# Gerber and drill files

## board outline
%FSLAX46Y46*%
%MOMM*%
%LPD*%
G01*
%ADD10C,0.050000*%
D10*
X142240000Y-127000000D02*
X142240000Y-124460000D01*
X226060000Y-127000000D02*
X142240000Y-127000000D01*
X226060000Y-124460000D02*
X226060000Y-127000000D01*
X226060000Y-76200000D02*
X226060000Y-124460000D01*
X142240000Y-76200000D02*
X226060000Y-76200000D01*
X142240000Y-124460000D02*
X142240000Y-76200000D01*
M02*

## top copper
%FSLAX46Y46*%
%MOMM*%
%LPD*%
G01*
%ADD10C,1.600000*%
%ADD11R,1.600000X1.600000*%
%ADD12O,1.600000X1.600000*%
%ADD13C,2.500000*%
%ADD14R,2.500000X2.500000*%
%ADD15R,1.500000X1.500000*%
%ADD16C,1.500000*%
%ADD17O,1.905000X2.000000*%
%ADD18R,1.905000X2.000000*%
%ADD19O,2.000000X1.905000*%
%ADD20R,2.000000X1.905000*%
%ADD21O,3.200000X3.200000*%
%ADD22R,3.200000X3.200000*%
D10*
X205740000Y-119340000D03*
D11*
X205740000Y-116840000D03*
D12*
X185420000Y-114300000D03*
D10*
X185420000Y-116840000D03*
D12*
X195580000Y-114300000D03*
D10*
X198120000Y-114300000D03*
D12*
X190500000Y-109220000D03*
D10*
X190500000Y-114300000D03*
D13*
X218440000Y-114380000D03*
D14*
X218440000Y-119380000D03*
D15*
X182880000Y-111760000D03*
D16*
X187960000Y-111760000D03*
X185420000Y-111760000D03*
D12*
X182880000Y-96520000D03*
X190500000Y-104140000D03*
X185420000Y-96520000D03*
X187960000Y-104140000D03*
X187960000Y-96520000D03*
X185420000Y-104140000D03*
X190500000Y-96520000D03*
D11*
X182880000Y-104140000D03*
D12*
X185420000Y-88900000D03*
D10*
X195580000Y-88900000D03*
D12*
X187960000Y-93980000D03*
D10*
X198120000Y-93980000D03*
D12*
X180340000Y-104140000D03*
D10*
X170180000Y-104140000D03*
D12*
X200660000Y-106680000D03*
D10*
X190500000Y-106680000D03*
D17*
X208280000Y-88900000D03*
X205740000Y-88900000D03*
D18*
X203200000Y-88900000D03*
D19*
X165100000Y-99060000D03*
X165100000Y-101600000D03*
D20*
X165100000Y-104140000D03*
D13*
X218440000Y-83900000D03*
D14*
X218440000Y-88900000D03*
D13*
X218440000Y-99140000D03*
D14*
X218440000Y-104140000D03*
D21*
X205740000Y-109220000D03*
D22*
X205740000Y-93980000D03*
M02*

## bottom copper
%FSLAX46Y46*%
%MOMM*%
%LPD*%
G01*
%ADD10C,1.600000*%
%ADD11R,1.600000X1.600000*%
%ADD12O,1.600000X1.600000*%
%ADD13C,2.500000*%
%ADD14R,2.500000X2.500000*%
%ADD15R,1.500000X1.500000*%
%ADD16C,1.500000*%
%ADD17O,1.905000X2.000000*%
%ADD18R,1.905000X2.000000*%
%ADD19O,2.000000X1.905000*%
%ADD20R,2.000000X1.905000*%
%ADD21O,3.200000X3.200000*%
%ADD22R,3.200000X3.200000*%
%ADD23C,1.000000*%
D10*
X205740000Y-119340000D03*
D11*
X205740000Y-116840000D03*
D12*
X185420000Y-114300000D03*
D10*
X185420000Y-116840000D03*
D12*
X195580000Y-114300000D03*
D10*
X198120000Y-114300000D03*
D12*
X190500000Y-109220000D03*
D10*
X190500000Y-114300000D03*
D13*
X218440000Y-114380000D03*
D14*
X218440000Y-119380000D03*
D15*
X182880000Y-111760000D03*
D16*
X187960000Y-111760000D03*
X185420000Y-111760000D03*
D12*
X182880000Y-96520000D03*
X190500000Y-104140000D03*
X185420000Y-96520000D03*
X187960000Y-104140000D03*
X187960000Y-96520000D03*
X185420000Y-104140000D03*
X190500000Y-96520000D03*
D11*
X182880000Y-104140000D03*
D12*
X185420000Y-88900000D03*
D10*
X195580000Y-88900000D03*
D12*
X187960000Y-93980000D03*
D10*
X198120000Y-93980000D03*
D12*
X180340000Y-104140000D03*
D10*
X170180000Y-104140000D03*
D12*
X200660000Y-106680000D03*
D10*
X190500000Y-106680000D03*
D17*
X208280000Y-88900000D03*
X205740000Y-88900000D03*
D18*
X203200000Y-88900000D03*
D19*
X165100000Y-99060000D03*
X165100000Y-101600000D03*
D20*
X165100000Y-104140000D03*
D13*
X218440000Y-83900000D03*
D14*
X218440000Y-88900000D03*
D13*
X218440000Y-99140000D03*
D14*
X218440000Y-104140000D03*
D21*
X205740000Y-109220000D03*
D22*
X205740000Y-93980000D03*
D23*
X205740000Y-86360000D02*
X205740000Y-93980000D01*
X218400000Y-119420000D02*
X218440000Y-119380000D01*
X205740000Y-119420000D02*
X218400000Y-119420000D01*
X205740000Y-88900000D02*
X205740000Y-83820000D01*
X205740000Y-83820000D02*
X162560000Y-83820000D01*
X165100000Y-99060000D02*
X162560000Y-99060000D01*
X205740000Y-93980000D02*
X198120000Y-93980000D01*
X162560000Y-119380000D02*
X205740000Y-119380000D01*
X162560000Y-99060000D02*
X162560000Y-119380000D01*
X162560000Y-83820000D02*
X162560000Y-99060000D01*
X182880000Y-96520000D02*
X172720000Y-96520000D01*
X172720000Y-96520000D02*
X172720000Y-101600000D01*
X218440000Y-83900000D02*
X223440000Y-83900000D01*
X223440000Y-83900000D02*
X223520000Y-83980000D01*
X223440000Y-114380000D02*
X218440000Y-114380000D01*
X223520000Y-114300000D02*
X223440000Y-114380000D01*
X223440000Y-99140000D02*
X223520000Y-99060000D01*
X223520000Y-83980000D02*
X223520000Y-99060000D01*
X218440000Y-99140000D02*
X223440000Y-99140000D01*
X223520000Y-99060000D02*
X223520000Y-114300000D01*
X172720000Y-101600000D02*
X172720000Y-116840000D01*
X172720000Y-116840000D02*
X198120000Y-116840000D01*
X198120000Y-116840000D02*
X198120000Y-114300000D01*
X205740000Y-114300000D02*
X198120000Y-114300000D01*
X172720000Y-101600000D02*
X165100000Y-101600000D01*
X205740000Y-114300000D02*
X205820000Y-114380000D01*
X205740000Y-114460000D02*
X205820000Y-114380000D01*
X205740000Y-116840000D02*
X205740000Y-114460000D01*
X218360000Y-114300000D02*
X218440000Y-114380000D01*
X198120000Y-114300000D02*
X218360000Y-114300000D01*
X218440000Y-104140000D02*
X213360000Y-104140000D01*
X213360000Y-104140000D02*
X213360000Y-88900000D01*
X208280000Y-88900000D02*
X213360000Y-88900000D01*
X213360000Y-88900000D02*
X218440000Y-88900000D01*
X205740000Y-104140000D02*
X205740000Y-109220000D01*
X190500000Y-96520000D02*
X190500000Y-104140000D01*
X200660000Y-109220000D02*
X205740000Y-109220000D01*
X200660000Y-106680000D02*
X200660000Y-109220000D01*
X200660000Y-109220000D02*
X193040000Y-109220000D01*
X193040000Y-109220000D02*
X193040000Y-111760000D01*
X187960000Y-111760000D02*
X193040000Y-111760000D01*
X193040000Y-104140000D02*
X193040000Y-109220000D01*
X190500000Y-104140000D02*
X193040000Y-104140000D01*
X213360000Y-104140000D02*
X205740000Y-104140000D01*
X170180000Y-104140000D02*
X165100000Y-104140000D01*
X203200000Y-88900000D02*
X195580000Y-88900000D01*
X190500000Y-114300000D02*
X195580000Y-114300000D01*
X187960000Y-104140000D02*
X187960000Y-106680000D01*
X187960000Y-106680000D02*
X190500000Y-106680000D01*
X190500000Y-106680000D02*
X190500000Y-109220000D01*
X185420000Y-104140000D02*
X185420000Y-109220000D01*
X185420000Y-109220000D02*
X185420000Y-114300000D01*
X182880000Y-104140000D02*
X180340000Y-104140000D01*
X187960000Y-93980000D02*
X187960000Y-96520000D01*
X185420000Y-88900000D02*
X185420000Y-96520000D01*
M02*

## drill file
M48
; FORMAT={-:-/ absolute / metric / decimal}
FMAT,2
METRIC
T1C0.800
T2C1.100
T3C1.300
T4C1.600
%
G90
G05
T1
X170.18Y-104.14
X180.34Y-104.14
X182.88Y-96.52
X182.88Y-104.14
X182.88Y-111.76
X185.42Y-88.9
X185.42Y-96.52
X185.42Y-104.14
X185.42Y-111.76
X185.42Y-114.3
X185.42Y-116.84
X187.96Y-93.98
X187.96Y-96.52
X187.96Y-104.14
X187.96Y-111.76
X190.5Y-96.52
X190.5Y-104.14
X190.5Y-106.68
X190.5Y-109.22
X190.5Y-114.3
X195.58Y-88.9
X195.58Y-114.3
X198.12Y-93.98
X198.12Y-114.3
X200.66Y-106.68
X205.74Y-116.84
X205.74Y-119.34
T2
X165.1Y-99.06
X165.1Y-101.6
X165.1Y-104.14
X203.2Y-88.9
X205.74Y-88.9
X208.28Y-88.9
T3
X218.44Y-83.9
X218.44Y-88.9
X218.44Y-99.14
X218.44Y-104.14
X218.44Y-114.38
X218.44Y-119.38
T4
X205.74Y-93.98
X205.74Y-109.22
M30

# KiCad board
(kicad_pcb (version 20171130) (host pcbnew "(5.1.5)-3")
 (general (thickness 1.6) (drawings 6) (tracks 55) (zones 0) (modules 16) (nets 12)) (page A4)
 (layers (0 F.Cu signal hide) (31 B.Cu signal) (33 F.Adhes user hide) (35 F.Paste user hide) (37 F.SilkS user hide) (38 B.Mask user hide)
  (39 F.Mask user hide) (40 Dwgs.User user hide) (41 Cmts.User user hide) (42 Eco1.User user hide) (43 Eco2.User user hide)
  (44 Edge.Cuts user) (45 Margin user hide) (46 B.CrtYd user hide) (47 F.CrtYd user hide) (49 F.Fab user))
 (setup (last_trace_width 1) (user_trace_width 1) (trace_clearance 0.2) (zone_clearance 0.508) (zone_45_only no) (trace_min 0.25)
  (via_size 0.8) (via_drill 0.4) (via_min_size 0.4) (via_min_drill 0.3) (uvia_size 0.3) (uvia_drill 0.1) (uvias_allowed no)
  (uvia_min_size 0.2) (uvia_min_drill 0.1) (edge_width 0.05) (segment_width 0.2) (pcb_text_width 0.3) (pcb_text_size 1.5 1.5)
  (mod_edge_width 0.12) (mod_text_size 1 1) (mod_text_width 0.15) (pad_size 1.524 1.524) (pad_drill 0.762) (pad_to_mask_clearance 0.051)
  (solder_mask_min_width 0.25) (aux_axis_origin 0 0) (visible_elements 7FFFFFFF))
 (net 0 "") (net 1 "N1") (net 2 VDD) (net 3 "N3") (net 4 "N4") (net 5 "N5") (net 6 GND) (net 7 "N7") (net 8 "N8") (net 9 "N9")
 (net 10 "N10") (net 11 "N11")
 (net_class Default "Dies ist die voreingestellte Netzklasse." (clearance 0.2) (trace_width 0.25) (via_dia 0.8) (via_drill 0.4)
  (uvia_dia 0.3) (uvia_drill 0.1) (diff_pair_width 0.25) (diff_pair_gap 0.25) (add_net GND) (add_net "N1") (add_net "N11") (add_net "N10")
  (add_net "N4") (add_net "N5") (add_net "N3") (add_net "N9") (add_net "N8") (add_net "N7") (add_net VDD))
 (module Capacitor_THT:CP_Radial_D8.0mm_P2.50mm (layer F.Cu) (at 205.74 116.84 270)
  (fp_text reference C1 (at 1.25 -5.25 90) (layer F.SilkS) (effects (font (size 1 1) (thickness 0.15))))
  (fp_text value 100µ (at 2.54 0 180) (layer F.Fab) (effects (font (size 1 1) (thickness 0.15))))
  (pad 2 thru_hole circle (at 2.5 0 270) (size 1.6 1.6) (drill 0.8) (layers *.Cu *.Mask) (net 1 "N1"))
  (pad 1 thru_hole rect (at 0 0 270) (size 1.6 1.6) (drill 0.8) (layers *.Cu *.Mask) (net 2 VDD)))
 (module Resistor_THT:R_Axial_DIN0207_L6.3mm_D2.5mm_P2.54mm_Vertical (layer F.Cu) (at 185.42 116.84 90)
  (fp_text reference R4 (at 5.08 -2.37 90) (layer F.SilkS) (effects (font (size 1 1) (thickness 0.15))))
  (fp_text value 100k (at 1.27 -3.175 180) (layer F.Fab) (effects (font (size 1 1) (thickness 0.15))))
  (pad 2 thru_hole oval (at 2.54 0 90) (size 1.6 1.6) (drill 0.8) (layers *.Cu *.Mask) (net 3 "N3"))
  (pad 1 thru_hole circle (at 0 0 90) (size 1.6 1.6) (drill 0.8) (layers *.Cu *.Mask) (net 2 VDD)))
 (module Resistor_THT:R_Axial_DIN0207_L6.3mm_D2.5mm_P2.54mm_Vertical (layer F.Cu) (at 198.12 114.3 180)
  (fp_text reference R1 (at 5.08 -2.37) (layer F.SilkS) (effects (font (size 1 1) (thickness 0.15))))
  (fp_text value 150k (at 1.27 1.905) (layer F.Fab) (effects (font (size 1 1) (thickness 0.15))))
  (pad 2 thru_hole oval (at 2.54 0 180) (size 1.6 1.6) (drill 0.8) (layers *.Cu *.Mask) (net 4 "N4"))
  (pad 1 thru_hole circle (at 0 0 180) (size 1.6 1.6) (drill 0.8) (layers *.Cu *.Mask) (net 2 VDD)))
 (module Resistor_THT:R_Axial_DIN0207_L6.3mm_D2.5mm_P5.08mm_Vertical (layer F.Cu) (at 190.5 114.3 90)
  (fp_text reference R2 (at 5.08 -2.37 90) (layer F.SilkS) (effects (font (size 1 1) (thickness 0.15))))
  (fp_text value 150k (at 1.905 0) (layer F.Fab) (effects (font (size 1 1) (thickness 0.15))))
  (pad 2 thru_hole oval (at 5.08 0 90) (size 1.6 1.6) (drill 0.8) (layers *.Cu *.Mask) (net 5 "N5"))
  (pad 1 thru_hole circle (at 0 0 90) (size 1.6 1.6) (drill 0.8) (layers *.Cu *.Mask) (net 4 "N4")))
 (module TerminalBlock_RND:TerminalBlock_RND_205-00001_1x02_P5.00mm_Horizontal (layer F.Cu) (at 218.44 119.38 90)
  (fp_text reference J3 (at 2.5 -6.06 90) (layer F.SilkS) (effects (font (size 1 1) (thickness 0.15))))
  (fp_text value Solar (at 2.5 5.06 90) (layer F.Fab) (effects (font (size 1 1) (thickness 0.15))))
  (pad 2 thru_hole circle (at 5 0 90) (size 2.5 2.5) (drill 1.3) (layers *.Cu *.Mask) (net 2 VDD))
  (pad 1 thru_hole rect (at 0 0 90) (size 2.5 2.5) (drill 1.3) (layers *.Cu *.Mask) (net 1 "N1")))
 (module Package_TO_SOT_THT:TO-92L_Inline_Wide (layer F.Cu) (at 182.88 111.76)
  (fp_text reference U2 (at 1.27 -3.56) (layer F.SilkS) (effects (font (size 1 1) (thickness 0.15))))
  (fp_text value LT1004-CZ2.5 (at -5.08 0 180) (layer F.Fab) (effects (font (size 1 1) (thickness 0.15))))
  (pad 1 thru_hole rect (at 0 0 90) (size 1.5 1.5) (drill 0.8) (layers *.Cu *.Mask))
  (pad 3 thru_hole circle (at 5.08 0 90) (size 1.5 1.5) (drill 0.8) (layers *.Cu *.Mask) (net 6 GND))
  (pad 2 thru_hole circle (at 2.54 0 90) (size 1.5 1.5) (drill 0.8) (layers *.Cu *.Mask) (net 3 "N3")))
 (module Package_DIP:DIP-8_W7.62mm (layer F.Cu) (at 182.88 104.14 90)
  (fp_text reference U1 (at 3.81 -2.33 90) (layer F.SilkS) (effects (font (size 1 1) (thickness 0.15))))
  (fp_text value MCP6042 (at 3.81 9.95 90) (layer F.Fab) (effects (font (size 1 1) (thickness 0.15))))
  (pad 8 thru_hole oval (at 7.62 0 90) (size 1.6 1.6) (drill 0.8) (layers *.Cu *.Mask) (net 2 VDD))
  (pad 4 thru_hole oval (at 0 7.62 90) (size 1.6 1.6) (drill 0.8) (layers *.Cu *.Mask) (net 6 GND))
  (pad 7 thru_hole oval (at 7.62 2.54 90) (size 1.6 1.6) (drill 0.8) (layers *.Cu *.Mask) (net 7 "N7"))
  (pad 3 thru_hole oval (at 0 5.08 90) (size 1.6 1.6) (drill 0.8) (layers *.Cu *.Mask) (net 5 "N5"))
  (pad 6 thru_hole oval (at 7.62 5.08 90) (size 1.6 1.6) (drill 0.8) (layers *.Cu *.Mask) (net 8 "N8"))
  (pad 2 thru_hole oval (at 0 2.54 90) (size 1.6 1.6) (drill 0.8) (layers *.Cu *.Mask) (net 3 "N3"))
  (pad 5 thru_hole oval (at 7.62 7.62 90) (size 1.6 1.6) (drill 0.8) (layers *.Cu *.Mask) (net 6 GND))
  (pad 1 thru_hole rect (at 0 0 90) (size 1.6 1.6) (drill 0.8) (layers *.Cu *.Mask) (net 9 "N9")))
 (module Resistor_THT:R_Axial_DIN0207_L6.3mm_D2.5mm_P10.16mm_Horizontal (layer F.Cu) (at 195.58 88.9 180)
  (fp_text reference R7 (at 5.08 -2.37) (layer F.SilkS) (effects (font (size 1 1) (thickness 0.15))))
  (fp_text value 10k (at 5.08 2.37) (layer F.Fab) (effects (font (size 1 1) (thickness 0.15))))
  (pad 2 thru_hole oval (at 10.16 0 180) (size 1.6 1.6) (drill 0.8) (layers *.Cu *.Mask) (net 7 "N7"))
  (pad 1 thru_hole circle (at 0 0 180) (size 1.6 1.6) (drill 0.8) (layers *.Cu *.Mask) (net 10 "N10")))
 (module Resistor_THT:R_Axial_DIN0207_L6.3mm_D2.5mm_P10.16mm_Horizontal (layer F.Cu) (at 198.12 93.98 180)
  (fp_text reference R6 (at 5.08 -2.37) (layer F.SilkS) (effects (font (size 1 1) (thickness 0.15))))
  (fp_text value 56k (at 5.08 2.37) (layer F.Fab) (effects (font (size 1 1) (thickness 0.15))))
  (pad 2 thru_hole oval (at 10.16 0 180) (size 1.6 1.6) (drill 0.8) (layers *.Cu *.Mask) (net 8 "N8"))
  (pad 1 thru_hole circle (at 0 0 180) (size 1.6 1.6) (drill 0.8) (layers *.Cu *.Mask) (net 1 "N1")))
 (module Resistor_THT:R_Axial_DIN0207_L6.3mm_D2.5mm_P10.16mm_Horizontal (layer F.Cu) (at 170.18 104.14)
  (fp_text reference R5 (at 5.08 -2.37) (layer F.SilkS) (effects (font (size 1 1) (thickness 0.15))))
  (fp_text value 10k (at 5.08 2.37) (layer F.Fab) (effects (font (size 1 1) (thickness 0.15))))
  (pad 2 thru_hole oval (at 10.16 0) (size 1.6 1.6) (drill 0.8) (layers *.Cu *.Mask) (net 9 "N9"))
  (pad 1 thru_hole circle (at 0 0) (size 1.6 1.6) (drill 0.8) (layers *.Cu *.Mask) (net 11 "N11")))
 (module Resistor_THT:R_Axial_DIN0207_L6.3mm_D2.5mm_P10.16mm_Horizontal (layer F.Cu) (at 190.5 106.68)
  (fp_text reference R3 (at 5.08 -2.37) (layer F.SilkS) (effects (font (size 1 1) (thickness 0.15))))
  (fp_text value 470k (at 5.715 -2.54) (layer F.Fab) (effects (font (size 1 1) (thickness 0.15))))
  (pad 2 thru_hole oval (at 10.16 0) (size 1.6 1.6) (drill 0.8) (layers *.Cu *.Mask) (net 6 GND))
  (pad 1 thru_hole circle (at 0 0) (size 1.6 1.6) (drill 0.8) (layers *.Cu *.Mask) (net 5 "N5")))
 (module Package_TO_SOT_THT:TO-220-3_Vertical (layer F.Cu) (at 203.2 88.9)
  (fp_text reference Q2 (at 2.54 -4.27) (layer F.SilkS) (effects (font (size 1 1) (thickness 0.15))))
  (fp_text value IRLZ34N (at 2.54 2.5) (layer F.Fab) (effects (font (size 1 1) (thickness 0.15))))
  (pad 3 thru_hole oval (at 5.08 0) (size 1.905 2) (drill 1.1) (layers *.Cu *.Mask) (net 6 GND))
  (pad 2 thru_hole oval (at 2.54 0) (size 1.905 2) (drill 1.1) (layers *.Cu *.Mask) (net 1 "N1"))
  (pad 1 thru_hole rect (at 0 0) (size 1.905 2) (drill 1.1) (layers *.Cu *.Mask) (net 10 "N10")))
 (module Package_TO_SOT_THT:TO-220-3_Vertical (layer F.Cu) (at 165.1 104.14 90)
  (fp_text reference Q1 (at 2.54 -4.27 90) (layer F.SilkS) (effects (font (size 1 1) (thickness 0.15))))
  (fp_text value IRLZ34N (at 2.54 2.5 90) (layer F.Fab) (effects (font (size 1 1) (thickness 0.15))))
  (pad 3 thru_hole oval (at 5.08 0 90) (size 1.905 2) (drill 1.1) (layers *.Cu *.Mask) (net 1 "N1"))
  (pad 2 thru_hole oval (at 2.54 0 90) (size 1.905 2) (drill 1.1) (layers *.Cu *.Mask) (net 2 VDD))
  (pad 1 thru_hole rect (at 0 0 90) (size 1.905 2) (drill 1.1) (layers *.Cu *.Mask) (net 11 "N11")))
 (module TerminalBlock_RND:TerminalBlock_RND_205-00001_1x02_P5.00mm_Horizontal (layer F.Cu) (at 218.44 88.9 90)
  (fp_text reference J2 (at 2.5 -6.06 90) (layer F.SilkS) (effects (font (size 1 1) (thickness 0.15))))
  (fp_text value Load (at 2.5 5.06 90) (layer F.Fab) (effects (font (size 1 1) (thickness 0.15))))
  (pad 2 thru_hole circle (at 5 0 90) (size 2.5 2.5) (drill 1.3) (layers *.Cu *.Mask) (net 2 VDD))
  (pad 1 thru_hole rect (at 0 0 90) (size 2.5 2.5) (drill 1.3) (layers *.Cu *.Mask) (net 6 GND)))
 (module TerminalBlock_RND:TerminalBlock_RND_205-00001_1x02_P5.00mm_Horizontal (layer F.Cu) (at 218.44 104.14 90)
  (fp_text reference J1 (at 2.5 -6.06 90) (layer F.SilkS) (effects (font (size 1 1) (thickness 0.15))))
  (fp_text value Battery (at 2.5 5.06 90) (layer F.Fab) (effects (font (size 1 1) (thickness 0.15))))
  (pad 2 thru_hole circle (at 5 0 90) (size 2.5 2.5) (drill 1.3) (layers *.Cu *.Mask) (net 2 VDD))
  (pad 1 thru_hole rect (at 0 0 90) (size 2.5 2.5) (drill 1.3) (layers *.Cu *.Mask) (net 6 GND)))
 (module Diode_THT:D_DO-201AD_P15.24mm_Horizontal (layer F.Cu) (at 205.74 93.98 270)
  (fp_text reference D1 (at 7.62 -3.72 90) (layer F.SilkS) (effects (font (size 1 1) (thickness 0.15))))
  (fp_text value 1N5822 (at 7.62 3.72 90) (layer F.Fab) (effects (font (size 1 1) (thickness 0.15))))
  (pad 2 thru_hole oval (at 15.24 0 270) (size 3.2 3.2) (drill 1.6) (layers *.Cu *.Mask) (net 6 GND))
  (pad 1 thru_hole rect (at 0 0 270) (size 3.2 3.2) (drill 1.6) (layers *.Cu *.Mask) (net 1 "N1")))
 (gr_line (start 142.24 127) (end 142.24 124.46) (layer Edge.Cuts) (width 0.05))
 (gr_line (start 226.06 127) (end 142.24 127) (layer Edge.Cuts) (width 0.05))
 (gr_line (start 226.06 124.46) (end 226.06 127) (layer Edge.Cuts) (width 0.05))
 (gr_line (start 226.06 76.2) (end 226.06 124.46) (layer Edge.Cuts) (width 0.05))
 (gr_line (start 142.24 76.2) (end 226.06 76.2) (layer Edge.Cuts) (width 0.05))
 (gr_line (start 142.24 124.46) (end 142.24 76.2) (layer Edge.Cuts) (width 0.05))
 (segment (start 205.74 86.36) (end 205.74 93.98) (width 1) (layer B.Cu) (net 1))
 (segment (start 218.4 119.42) (end 218.44 119.38) (width 1) (layer B.Cu) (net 1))
 (segment (start 205.74 119.42) (end 218.4 119.42) (width 1) (layer B.Cu) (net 1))
 (segment (start 205.74 88.9) (end 205.74 83.82) (width 1) (layer B.Cu) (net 1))
 (segment (start 205.74 83.82) (end 162.56 83.82) (width 1) (layer B.Cu) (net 1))
 (segment (start 165.1 99.06) (end 162.56 99.06) (width 1) (layer B.Cu) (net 1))
 (segment (start 205.74 93.98) (end 198.12 93.98) (width 1) (layer B.Cu) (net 1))
 (segment (start 162.56 119.38) (end 205.74 119.38) (width 1) (layer B.Cu) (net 1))
 (segment (start 162.56 99.06) (end 162.56 119.38) (width 1) (layer B.Cu) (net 1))
 (segment (start 162.56 83.82) (end 162.56 99.06) (width 1) (layer B.Cu) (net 1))
 (segment (start 182.88 96.52) (end 172.72 96.52) (width 1) (layer B.Cu) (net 2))
 (segment (start 172.72 96.52) (end 172.72 101.6) (width 1) (layer B.Cu) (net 2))
 (segment (start 218.44 83.9) (end 223.44 83.9) (width 1) (layer B.Cu) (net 2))
 (segment (start 223.44 83.9) (end 223.52 83.98) (width 1) (layer B.Cu) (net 2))
 (segment (start 223.44 114.38) (end 218.44 114.38) (width 1) (layer B.Cu) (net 2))
 (segment (start 223.52 114.3) (end 223.44 114.38) (width 1) (layer B.Cu) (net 2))
 (segment (start 223.44 99.14) (end 223.52 99.06) (width 1) (layer B.Cu) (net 2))
 (segment (start 223.52 83.98) (end 223.52 99.06) (width 1) (layer B.Cu) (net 2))
 (segment (start 218.44 99.14) (end 223.44 99.14) (width 1) (layer B.Cu) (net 2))
 (segment (start 223.52 99.06) (end 223.52 114.3) (width 1) (layer B.Cu) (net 2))
 (segment (start 172.72 101.6) (end 172.72 116.84) (width 1) (layer B.Cu) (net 2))
 (segment (start 172.72 116.84) (end 198.12 116.84) (width 1) (layer B.Cu) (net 2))
 (segment (start 198.12 116.84) (end 198.12 114.3) (width 1) (layer B.Cu) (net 2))
 (segment (start 205.74 114.3) (end 198.12 114.3) (width 1) (layer B.Cu) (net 2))
 (segment (start 172.72 101.6) (end 165.1 101.6) (width 1) (layer B.Cu) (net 2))
 (segment (start 205.74 114.3) (end 205.82 114.38) (width 1) (layer B.Cu) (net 2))
 (segment (start 205.74 114.46) (end 205.82 114.38) (width 1) (layer B.Cu) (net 2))
 (segment (start 205.74 116.84) (end 205.74 114.46) (width 1) (layer B.Cu) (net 2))
 (segment (start 218.36 114.3) (end 218.44 114.38) (width 1) (layer B.Cu) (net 2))
 (segment (start 198.12 114.3) (end 218.36 114.3) (width 1) (layer B.Cu) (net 2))
 (segment (start 218.44 104.14) (end 213.36 104.14) (width 1) (layer B.Cu) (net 6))
 (segment (start 213.36 104.14) (end 213.36 88.9) (width 1) (layer B.Cu) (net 6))
 (segment (start 208.28 88.9) (end 213.36 88.9) (width 1) (layer B.Cu) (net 6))
 (segment (start 213.36 88.9) (end 218.44 88.9) (width 1) (layer B.Cu) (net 6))
 (segment (start 205.74 104.14) (end 205.74 109.22) (width 1) (layer B.Cu) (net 6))
 (segment (start 190.5 96.52) (end 190.5 104.14) (width 1) (layer B.Cu) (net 6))
 (segment (start 200.66 109.22) (end 205.74 109.22) (width 1) (layer B.Cu) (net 6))
 (segment (start 200.66 106.68) (end 200.66 109.22) (width 1) (layer B.Cu) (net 6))
 (segment (start 200.66 109.22) (end 193.04 109.22) (width 1) (layer B.Cu) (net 6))
 (segment (start 193.04 109.22) (end 193.04 111.76) (width 1) (layer B.Cu) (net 6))
 (segment (start 187.96 111.76) (end 193.04 111.76) (width 1) (layer B.Cu) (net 6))
 (segment (start 193.04 104.14) (end 193.04 109.22) (width 1) (layer B.Cu) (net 6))
 (segment (start 190.5 104.14) (end 193.04 104.14) (width 1) (layer B.Cu) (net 6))
 (segment (start 213.36 104.14) (end 205.74 104.14) (width 1) (layer B.Cu) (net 6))
 (segment (start 170.18 104.14) (end 165.1 104.14) (width 1) (layer B.Cu) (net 11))
 (segment (start 203.2 88.9) (end 195.58 88.9) (width 1) (layer B.Cu) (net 10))
 (segment (start 190.5 114.3) (end 195.58 114.3) (width 1) (layer B.Cu) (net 4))
 (segment (start 187.96 104.14) (end 187.96 106.68) (width 1) (layer B.Cu) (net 5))
 (segment (start 187.96 106.68) (end 190.5 106.68) (width 1) (layer B.Cu) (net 5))
 (segment (start 190.5 106.68) (end 190.5 109.22) (width 1) (layer B.Cu) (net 5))
 (segment (start 185.42 104.14) (end 185.42 109.22) (width 1) (layer B.Cu) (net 3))
 (segment (start 185.42 109.22) (end 185.42 114.3) (width 1) (layer B.Cu) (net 3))
 (segment (start 182.88 104.14) (end 180.34 104.14) (width 1) (layer B.Cu) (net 9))
 (segment (start 187.96 93.98) (end 187.96 96.52) (width 1) (layer B.Cu) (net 8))
 (segment (start 185.42 88.9) (end 185.42 96.52) (width 1) (layer B.Cu) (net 7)))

